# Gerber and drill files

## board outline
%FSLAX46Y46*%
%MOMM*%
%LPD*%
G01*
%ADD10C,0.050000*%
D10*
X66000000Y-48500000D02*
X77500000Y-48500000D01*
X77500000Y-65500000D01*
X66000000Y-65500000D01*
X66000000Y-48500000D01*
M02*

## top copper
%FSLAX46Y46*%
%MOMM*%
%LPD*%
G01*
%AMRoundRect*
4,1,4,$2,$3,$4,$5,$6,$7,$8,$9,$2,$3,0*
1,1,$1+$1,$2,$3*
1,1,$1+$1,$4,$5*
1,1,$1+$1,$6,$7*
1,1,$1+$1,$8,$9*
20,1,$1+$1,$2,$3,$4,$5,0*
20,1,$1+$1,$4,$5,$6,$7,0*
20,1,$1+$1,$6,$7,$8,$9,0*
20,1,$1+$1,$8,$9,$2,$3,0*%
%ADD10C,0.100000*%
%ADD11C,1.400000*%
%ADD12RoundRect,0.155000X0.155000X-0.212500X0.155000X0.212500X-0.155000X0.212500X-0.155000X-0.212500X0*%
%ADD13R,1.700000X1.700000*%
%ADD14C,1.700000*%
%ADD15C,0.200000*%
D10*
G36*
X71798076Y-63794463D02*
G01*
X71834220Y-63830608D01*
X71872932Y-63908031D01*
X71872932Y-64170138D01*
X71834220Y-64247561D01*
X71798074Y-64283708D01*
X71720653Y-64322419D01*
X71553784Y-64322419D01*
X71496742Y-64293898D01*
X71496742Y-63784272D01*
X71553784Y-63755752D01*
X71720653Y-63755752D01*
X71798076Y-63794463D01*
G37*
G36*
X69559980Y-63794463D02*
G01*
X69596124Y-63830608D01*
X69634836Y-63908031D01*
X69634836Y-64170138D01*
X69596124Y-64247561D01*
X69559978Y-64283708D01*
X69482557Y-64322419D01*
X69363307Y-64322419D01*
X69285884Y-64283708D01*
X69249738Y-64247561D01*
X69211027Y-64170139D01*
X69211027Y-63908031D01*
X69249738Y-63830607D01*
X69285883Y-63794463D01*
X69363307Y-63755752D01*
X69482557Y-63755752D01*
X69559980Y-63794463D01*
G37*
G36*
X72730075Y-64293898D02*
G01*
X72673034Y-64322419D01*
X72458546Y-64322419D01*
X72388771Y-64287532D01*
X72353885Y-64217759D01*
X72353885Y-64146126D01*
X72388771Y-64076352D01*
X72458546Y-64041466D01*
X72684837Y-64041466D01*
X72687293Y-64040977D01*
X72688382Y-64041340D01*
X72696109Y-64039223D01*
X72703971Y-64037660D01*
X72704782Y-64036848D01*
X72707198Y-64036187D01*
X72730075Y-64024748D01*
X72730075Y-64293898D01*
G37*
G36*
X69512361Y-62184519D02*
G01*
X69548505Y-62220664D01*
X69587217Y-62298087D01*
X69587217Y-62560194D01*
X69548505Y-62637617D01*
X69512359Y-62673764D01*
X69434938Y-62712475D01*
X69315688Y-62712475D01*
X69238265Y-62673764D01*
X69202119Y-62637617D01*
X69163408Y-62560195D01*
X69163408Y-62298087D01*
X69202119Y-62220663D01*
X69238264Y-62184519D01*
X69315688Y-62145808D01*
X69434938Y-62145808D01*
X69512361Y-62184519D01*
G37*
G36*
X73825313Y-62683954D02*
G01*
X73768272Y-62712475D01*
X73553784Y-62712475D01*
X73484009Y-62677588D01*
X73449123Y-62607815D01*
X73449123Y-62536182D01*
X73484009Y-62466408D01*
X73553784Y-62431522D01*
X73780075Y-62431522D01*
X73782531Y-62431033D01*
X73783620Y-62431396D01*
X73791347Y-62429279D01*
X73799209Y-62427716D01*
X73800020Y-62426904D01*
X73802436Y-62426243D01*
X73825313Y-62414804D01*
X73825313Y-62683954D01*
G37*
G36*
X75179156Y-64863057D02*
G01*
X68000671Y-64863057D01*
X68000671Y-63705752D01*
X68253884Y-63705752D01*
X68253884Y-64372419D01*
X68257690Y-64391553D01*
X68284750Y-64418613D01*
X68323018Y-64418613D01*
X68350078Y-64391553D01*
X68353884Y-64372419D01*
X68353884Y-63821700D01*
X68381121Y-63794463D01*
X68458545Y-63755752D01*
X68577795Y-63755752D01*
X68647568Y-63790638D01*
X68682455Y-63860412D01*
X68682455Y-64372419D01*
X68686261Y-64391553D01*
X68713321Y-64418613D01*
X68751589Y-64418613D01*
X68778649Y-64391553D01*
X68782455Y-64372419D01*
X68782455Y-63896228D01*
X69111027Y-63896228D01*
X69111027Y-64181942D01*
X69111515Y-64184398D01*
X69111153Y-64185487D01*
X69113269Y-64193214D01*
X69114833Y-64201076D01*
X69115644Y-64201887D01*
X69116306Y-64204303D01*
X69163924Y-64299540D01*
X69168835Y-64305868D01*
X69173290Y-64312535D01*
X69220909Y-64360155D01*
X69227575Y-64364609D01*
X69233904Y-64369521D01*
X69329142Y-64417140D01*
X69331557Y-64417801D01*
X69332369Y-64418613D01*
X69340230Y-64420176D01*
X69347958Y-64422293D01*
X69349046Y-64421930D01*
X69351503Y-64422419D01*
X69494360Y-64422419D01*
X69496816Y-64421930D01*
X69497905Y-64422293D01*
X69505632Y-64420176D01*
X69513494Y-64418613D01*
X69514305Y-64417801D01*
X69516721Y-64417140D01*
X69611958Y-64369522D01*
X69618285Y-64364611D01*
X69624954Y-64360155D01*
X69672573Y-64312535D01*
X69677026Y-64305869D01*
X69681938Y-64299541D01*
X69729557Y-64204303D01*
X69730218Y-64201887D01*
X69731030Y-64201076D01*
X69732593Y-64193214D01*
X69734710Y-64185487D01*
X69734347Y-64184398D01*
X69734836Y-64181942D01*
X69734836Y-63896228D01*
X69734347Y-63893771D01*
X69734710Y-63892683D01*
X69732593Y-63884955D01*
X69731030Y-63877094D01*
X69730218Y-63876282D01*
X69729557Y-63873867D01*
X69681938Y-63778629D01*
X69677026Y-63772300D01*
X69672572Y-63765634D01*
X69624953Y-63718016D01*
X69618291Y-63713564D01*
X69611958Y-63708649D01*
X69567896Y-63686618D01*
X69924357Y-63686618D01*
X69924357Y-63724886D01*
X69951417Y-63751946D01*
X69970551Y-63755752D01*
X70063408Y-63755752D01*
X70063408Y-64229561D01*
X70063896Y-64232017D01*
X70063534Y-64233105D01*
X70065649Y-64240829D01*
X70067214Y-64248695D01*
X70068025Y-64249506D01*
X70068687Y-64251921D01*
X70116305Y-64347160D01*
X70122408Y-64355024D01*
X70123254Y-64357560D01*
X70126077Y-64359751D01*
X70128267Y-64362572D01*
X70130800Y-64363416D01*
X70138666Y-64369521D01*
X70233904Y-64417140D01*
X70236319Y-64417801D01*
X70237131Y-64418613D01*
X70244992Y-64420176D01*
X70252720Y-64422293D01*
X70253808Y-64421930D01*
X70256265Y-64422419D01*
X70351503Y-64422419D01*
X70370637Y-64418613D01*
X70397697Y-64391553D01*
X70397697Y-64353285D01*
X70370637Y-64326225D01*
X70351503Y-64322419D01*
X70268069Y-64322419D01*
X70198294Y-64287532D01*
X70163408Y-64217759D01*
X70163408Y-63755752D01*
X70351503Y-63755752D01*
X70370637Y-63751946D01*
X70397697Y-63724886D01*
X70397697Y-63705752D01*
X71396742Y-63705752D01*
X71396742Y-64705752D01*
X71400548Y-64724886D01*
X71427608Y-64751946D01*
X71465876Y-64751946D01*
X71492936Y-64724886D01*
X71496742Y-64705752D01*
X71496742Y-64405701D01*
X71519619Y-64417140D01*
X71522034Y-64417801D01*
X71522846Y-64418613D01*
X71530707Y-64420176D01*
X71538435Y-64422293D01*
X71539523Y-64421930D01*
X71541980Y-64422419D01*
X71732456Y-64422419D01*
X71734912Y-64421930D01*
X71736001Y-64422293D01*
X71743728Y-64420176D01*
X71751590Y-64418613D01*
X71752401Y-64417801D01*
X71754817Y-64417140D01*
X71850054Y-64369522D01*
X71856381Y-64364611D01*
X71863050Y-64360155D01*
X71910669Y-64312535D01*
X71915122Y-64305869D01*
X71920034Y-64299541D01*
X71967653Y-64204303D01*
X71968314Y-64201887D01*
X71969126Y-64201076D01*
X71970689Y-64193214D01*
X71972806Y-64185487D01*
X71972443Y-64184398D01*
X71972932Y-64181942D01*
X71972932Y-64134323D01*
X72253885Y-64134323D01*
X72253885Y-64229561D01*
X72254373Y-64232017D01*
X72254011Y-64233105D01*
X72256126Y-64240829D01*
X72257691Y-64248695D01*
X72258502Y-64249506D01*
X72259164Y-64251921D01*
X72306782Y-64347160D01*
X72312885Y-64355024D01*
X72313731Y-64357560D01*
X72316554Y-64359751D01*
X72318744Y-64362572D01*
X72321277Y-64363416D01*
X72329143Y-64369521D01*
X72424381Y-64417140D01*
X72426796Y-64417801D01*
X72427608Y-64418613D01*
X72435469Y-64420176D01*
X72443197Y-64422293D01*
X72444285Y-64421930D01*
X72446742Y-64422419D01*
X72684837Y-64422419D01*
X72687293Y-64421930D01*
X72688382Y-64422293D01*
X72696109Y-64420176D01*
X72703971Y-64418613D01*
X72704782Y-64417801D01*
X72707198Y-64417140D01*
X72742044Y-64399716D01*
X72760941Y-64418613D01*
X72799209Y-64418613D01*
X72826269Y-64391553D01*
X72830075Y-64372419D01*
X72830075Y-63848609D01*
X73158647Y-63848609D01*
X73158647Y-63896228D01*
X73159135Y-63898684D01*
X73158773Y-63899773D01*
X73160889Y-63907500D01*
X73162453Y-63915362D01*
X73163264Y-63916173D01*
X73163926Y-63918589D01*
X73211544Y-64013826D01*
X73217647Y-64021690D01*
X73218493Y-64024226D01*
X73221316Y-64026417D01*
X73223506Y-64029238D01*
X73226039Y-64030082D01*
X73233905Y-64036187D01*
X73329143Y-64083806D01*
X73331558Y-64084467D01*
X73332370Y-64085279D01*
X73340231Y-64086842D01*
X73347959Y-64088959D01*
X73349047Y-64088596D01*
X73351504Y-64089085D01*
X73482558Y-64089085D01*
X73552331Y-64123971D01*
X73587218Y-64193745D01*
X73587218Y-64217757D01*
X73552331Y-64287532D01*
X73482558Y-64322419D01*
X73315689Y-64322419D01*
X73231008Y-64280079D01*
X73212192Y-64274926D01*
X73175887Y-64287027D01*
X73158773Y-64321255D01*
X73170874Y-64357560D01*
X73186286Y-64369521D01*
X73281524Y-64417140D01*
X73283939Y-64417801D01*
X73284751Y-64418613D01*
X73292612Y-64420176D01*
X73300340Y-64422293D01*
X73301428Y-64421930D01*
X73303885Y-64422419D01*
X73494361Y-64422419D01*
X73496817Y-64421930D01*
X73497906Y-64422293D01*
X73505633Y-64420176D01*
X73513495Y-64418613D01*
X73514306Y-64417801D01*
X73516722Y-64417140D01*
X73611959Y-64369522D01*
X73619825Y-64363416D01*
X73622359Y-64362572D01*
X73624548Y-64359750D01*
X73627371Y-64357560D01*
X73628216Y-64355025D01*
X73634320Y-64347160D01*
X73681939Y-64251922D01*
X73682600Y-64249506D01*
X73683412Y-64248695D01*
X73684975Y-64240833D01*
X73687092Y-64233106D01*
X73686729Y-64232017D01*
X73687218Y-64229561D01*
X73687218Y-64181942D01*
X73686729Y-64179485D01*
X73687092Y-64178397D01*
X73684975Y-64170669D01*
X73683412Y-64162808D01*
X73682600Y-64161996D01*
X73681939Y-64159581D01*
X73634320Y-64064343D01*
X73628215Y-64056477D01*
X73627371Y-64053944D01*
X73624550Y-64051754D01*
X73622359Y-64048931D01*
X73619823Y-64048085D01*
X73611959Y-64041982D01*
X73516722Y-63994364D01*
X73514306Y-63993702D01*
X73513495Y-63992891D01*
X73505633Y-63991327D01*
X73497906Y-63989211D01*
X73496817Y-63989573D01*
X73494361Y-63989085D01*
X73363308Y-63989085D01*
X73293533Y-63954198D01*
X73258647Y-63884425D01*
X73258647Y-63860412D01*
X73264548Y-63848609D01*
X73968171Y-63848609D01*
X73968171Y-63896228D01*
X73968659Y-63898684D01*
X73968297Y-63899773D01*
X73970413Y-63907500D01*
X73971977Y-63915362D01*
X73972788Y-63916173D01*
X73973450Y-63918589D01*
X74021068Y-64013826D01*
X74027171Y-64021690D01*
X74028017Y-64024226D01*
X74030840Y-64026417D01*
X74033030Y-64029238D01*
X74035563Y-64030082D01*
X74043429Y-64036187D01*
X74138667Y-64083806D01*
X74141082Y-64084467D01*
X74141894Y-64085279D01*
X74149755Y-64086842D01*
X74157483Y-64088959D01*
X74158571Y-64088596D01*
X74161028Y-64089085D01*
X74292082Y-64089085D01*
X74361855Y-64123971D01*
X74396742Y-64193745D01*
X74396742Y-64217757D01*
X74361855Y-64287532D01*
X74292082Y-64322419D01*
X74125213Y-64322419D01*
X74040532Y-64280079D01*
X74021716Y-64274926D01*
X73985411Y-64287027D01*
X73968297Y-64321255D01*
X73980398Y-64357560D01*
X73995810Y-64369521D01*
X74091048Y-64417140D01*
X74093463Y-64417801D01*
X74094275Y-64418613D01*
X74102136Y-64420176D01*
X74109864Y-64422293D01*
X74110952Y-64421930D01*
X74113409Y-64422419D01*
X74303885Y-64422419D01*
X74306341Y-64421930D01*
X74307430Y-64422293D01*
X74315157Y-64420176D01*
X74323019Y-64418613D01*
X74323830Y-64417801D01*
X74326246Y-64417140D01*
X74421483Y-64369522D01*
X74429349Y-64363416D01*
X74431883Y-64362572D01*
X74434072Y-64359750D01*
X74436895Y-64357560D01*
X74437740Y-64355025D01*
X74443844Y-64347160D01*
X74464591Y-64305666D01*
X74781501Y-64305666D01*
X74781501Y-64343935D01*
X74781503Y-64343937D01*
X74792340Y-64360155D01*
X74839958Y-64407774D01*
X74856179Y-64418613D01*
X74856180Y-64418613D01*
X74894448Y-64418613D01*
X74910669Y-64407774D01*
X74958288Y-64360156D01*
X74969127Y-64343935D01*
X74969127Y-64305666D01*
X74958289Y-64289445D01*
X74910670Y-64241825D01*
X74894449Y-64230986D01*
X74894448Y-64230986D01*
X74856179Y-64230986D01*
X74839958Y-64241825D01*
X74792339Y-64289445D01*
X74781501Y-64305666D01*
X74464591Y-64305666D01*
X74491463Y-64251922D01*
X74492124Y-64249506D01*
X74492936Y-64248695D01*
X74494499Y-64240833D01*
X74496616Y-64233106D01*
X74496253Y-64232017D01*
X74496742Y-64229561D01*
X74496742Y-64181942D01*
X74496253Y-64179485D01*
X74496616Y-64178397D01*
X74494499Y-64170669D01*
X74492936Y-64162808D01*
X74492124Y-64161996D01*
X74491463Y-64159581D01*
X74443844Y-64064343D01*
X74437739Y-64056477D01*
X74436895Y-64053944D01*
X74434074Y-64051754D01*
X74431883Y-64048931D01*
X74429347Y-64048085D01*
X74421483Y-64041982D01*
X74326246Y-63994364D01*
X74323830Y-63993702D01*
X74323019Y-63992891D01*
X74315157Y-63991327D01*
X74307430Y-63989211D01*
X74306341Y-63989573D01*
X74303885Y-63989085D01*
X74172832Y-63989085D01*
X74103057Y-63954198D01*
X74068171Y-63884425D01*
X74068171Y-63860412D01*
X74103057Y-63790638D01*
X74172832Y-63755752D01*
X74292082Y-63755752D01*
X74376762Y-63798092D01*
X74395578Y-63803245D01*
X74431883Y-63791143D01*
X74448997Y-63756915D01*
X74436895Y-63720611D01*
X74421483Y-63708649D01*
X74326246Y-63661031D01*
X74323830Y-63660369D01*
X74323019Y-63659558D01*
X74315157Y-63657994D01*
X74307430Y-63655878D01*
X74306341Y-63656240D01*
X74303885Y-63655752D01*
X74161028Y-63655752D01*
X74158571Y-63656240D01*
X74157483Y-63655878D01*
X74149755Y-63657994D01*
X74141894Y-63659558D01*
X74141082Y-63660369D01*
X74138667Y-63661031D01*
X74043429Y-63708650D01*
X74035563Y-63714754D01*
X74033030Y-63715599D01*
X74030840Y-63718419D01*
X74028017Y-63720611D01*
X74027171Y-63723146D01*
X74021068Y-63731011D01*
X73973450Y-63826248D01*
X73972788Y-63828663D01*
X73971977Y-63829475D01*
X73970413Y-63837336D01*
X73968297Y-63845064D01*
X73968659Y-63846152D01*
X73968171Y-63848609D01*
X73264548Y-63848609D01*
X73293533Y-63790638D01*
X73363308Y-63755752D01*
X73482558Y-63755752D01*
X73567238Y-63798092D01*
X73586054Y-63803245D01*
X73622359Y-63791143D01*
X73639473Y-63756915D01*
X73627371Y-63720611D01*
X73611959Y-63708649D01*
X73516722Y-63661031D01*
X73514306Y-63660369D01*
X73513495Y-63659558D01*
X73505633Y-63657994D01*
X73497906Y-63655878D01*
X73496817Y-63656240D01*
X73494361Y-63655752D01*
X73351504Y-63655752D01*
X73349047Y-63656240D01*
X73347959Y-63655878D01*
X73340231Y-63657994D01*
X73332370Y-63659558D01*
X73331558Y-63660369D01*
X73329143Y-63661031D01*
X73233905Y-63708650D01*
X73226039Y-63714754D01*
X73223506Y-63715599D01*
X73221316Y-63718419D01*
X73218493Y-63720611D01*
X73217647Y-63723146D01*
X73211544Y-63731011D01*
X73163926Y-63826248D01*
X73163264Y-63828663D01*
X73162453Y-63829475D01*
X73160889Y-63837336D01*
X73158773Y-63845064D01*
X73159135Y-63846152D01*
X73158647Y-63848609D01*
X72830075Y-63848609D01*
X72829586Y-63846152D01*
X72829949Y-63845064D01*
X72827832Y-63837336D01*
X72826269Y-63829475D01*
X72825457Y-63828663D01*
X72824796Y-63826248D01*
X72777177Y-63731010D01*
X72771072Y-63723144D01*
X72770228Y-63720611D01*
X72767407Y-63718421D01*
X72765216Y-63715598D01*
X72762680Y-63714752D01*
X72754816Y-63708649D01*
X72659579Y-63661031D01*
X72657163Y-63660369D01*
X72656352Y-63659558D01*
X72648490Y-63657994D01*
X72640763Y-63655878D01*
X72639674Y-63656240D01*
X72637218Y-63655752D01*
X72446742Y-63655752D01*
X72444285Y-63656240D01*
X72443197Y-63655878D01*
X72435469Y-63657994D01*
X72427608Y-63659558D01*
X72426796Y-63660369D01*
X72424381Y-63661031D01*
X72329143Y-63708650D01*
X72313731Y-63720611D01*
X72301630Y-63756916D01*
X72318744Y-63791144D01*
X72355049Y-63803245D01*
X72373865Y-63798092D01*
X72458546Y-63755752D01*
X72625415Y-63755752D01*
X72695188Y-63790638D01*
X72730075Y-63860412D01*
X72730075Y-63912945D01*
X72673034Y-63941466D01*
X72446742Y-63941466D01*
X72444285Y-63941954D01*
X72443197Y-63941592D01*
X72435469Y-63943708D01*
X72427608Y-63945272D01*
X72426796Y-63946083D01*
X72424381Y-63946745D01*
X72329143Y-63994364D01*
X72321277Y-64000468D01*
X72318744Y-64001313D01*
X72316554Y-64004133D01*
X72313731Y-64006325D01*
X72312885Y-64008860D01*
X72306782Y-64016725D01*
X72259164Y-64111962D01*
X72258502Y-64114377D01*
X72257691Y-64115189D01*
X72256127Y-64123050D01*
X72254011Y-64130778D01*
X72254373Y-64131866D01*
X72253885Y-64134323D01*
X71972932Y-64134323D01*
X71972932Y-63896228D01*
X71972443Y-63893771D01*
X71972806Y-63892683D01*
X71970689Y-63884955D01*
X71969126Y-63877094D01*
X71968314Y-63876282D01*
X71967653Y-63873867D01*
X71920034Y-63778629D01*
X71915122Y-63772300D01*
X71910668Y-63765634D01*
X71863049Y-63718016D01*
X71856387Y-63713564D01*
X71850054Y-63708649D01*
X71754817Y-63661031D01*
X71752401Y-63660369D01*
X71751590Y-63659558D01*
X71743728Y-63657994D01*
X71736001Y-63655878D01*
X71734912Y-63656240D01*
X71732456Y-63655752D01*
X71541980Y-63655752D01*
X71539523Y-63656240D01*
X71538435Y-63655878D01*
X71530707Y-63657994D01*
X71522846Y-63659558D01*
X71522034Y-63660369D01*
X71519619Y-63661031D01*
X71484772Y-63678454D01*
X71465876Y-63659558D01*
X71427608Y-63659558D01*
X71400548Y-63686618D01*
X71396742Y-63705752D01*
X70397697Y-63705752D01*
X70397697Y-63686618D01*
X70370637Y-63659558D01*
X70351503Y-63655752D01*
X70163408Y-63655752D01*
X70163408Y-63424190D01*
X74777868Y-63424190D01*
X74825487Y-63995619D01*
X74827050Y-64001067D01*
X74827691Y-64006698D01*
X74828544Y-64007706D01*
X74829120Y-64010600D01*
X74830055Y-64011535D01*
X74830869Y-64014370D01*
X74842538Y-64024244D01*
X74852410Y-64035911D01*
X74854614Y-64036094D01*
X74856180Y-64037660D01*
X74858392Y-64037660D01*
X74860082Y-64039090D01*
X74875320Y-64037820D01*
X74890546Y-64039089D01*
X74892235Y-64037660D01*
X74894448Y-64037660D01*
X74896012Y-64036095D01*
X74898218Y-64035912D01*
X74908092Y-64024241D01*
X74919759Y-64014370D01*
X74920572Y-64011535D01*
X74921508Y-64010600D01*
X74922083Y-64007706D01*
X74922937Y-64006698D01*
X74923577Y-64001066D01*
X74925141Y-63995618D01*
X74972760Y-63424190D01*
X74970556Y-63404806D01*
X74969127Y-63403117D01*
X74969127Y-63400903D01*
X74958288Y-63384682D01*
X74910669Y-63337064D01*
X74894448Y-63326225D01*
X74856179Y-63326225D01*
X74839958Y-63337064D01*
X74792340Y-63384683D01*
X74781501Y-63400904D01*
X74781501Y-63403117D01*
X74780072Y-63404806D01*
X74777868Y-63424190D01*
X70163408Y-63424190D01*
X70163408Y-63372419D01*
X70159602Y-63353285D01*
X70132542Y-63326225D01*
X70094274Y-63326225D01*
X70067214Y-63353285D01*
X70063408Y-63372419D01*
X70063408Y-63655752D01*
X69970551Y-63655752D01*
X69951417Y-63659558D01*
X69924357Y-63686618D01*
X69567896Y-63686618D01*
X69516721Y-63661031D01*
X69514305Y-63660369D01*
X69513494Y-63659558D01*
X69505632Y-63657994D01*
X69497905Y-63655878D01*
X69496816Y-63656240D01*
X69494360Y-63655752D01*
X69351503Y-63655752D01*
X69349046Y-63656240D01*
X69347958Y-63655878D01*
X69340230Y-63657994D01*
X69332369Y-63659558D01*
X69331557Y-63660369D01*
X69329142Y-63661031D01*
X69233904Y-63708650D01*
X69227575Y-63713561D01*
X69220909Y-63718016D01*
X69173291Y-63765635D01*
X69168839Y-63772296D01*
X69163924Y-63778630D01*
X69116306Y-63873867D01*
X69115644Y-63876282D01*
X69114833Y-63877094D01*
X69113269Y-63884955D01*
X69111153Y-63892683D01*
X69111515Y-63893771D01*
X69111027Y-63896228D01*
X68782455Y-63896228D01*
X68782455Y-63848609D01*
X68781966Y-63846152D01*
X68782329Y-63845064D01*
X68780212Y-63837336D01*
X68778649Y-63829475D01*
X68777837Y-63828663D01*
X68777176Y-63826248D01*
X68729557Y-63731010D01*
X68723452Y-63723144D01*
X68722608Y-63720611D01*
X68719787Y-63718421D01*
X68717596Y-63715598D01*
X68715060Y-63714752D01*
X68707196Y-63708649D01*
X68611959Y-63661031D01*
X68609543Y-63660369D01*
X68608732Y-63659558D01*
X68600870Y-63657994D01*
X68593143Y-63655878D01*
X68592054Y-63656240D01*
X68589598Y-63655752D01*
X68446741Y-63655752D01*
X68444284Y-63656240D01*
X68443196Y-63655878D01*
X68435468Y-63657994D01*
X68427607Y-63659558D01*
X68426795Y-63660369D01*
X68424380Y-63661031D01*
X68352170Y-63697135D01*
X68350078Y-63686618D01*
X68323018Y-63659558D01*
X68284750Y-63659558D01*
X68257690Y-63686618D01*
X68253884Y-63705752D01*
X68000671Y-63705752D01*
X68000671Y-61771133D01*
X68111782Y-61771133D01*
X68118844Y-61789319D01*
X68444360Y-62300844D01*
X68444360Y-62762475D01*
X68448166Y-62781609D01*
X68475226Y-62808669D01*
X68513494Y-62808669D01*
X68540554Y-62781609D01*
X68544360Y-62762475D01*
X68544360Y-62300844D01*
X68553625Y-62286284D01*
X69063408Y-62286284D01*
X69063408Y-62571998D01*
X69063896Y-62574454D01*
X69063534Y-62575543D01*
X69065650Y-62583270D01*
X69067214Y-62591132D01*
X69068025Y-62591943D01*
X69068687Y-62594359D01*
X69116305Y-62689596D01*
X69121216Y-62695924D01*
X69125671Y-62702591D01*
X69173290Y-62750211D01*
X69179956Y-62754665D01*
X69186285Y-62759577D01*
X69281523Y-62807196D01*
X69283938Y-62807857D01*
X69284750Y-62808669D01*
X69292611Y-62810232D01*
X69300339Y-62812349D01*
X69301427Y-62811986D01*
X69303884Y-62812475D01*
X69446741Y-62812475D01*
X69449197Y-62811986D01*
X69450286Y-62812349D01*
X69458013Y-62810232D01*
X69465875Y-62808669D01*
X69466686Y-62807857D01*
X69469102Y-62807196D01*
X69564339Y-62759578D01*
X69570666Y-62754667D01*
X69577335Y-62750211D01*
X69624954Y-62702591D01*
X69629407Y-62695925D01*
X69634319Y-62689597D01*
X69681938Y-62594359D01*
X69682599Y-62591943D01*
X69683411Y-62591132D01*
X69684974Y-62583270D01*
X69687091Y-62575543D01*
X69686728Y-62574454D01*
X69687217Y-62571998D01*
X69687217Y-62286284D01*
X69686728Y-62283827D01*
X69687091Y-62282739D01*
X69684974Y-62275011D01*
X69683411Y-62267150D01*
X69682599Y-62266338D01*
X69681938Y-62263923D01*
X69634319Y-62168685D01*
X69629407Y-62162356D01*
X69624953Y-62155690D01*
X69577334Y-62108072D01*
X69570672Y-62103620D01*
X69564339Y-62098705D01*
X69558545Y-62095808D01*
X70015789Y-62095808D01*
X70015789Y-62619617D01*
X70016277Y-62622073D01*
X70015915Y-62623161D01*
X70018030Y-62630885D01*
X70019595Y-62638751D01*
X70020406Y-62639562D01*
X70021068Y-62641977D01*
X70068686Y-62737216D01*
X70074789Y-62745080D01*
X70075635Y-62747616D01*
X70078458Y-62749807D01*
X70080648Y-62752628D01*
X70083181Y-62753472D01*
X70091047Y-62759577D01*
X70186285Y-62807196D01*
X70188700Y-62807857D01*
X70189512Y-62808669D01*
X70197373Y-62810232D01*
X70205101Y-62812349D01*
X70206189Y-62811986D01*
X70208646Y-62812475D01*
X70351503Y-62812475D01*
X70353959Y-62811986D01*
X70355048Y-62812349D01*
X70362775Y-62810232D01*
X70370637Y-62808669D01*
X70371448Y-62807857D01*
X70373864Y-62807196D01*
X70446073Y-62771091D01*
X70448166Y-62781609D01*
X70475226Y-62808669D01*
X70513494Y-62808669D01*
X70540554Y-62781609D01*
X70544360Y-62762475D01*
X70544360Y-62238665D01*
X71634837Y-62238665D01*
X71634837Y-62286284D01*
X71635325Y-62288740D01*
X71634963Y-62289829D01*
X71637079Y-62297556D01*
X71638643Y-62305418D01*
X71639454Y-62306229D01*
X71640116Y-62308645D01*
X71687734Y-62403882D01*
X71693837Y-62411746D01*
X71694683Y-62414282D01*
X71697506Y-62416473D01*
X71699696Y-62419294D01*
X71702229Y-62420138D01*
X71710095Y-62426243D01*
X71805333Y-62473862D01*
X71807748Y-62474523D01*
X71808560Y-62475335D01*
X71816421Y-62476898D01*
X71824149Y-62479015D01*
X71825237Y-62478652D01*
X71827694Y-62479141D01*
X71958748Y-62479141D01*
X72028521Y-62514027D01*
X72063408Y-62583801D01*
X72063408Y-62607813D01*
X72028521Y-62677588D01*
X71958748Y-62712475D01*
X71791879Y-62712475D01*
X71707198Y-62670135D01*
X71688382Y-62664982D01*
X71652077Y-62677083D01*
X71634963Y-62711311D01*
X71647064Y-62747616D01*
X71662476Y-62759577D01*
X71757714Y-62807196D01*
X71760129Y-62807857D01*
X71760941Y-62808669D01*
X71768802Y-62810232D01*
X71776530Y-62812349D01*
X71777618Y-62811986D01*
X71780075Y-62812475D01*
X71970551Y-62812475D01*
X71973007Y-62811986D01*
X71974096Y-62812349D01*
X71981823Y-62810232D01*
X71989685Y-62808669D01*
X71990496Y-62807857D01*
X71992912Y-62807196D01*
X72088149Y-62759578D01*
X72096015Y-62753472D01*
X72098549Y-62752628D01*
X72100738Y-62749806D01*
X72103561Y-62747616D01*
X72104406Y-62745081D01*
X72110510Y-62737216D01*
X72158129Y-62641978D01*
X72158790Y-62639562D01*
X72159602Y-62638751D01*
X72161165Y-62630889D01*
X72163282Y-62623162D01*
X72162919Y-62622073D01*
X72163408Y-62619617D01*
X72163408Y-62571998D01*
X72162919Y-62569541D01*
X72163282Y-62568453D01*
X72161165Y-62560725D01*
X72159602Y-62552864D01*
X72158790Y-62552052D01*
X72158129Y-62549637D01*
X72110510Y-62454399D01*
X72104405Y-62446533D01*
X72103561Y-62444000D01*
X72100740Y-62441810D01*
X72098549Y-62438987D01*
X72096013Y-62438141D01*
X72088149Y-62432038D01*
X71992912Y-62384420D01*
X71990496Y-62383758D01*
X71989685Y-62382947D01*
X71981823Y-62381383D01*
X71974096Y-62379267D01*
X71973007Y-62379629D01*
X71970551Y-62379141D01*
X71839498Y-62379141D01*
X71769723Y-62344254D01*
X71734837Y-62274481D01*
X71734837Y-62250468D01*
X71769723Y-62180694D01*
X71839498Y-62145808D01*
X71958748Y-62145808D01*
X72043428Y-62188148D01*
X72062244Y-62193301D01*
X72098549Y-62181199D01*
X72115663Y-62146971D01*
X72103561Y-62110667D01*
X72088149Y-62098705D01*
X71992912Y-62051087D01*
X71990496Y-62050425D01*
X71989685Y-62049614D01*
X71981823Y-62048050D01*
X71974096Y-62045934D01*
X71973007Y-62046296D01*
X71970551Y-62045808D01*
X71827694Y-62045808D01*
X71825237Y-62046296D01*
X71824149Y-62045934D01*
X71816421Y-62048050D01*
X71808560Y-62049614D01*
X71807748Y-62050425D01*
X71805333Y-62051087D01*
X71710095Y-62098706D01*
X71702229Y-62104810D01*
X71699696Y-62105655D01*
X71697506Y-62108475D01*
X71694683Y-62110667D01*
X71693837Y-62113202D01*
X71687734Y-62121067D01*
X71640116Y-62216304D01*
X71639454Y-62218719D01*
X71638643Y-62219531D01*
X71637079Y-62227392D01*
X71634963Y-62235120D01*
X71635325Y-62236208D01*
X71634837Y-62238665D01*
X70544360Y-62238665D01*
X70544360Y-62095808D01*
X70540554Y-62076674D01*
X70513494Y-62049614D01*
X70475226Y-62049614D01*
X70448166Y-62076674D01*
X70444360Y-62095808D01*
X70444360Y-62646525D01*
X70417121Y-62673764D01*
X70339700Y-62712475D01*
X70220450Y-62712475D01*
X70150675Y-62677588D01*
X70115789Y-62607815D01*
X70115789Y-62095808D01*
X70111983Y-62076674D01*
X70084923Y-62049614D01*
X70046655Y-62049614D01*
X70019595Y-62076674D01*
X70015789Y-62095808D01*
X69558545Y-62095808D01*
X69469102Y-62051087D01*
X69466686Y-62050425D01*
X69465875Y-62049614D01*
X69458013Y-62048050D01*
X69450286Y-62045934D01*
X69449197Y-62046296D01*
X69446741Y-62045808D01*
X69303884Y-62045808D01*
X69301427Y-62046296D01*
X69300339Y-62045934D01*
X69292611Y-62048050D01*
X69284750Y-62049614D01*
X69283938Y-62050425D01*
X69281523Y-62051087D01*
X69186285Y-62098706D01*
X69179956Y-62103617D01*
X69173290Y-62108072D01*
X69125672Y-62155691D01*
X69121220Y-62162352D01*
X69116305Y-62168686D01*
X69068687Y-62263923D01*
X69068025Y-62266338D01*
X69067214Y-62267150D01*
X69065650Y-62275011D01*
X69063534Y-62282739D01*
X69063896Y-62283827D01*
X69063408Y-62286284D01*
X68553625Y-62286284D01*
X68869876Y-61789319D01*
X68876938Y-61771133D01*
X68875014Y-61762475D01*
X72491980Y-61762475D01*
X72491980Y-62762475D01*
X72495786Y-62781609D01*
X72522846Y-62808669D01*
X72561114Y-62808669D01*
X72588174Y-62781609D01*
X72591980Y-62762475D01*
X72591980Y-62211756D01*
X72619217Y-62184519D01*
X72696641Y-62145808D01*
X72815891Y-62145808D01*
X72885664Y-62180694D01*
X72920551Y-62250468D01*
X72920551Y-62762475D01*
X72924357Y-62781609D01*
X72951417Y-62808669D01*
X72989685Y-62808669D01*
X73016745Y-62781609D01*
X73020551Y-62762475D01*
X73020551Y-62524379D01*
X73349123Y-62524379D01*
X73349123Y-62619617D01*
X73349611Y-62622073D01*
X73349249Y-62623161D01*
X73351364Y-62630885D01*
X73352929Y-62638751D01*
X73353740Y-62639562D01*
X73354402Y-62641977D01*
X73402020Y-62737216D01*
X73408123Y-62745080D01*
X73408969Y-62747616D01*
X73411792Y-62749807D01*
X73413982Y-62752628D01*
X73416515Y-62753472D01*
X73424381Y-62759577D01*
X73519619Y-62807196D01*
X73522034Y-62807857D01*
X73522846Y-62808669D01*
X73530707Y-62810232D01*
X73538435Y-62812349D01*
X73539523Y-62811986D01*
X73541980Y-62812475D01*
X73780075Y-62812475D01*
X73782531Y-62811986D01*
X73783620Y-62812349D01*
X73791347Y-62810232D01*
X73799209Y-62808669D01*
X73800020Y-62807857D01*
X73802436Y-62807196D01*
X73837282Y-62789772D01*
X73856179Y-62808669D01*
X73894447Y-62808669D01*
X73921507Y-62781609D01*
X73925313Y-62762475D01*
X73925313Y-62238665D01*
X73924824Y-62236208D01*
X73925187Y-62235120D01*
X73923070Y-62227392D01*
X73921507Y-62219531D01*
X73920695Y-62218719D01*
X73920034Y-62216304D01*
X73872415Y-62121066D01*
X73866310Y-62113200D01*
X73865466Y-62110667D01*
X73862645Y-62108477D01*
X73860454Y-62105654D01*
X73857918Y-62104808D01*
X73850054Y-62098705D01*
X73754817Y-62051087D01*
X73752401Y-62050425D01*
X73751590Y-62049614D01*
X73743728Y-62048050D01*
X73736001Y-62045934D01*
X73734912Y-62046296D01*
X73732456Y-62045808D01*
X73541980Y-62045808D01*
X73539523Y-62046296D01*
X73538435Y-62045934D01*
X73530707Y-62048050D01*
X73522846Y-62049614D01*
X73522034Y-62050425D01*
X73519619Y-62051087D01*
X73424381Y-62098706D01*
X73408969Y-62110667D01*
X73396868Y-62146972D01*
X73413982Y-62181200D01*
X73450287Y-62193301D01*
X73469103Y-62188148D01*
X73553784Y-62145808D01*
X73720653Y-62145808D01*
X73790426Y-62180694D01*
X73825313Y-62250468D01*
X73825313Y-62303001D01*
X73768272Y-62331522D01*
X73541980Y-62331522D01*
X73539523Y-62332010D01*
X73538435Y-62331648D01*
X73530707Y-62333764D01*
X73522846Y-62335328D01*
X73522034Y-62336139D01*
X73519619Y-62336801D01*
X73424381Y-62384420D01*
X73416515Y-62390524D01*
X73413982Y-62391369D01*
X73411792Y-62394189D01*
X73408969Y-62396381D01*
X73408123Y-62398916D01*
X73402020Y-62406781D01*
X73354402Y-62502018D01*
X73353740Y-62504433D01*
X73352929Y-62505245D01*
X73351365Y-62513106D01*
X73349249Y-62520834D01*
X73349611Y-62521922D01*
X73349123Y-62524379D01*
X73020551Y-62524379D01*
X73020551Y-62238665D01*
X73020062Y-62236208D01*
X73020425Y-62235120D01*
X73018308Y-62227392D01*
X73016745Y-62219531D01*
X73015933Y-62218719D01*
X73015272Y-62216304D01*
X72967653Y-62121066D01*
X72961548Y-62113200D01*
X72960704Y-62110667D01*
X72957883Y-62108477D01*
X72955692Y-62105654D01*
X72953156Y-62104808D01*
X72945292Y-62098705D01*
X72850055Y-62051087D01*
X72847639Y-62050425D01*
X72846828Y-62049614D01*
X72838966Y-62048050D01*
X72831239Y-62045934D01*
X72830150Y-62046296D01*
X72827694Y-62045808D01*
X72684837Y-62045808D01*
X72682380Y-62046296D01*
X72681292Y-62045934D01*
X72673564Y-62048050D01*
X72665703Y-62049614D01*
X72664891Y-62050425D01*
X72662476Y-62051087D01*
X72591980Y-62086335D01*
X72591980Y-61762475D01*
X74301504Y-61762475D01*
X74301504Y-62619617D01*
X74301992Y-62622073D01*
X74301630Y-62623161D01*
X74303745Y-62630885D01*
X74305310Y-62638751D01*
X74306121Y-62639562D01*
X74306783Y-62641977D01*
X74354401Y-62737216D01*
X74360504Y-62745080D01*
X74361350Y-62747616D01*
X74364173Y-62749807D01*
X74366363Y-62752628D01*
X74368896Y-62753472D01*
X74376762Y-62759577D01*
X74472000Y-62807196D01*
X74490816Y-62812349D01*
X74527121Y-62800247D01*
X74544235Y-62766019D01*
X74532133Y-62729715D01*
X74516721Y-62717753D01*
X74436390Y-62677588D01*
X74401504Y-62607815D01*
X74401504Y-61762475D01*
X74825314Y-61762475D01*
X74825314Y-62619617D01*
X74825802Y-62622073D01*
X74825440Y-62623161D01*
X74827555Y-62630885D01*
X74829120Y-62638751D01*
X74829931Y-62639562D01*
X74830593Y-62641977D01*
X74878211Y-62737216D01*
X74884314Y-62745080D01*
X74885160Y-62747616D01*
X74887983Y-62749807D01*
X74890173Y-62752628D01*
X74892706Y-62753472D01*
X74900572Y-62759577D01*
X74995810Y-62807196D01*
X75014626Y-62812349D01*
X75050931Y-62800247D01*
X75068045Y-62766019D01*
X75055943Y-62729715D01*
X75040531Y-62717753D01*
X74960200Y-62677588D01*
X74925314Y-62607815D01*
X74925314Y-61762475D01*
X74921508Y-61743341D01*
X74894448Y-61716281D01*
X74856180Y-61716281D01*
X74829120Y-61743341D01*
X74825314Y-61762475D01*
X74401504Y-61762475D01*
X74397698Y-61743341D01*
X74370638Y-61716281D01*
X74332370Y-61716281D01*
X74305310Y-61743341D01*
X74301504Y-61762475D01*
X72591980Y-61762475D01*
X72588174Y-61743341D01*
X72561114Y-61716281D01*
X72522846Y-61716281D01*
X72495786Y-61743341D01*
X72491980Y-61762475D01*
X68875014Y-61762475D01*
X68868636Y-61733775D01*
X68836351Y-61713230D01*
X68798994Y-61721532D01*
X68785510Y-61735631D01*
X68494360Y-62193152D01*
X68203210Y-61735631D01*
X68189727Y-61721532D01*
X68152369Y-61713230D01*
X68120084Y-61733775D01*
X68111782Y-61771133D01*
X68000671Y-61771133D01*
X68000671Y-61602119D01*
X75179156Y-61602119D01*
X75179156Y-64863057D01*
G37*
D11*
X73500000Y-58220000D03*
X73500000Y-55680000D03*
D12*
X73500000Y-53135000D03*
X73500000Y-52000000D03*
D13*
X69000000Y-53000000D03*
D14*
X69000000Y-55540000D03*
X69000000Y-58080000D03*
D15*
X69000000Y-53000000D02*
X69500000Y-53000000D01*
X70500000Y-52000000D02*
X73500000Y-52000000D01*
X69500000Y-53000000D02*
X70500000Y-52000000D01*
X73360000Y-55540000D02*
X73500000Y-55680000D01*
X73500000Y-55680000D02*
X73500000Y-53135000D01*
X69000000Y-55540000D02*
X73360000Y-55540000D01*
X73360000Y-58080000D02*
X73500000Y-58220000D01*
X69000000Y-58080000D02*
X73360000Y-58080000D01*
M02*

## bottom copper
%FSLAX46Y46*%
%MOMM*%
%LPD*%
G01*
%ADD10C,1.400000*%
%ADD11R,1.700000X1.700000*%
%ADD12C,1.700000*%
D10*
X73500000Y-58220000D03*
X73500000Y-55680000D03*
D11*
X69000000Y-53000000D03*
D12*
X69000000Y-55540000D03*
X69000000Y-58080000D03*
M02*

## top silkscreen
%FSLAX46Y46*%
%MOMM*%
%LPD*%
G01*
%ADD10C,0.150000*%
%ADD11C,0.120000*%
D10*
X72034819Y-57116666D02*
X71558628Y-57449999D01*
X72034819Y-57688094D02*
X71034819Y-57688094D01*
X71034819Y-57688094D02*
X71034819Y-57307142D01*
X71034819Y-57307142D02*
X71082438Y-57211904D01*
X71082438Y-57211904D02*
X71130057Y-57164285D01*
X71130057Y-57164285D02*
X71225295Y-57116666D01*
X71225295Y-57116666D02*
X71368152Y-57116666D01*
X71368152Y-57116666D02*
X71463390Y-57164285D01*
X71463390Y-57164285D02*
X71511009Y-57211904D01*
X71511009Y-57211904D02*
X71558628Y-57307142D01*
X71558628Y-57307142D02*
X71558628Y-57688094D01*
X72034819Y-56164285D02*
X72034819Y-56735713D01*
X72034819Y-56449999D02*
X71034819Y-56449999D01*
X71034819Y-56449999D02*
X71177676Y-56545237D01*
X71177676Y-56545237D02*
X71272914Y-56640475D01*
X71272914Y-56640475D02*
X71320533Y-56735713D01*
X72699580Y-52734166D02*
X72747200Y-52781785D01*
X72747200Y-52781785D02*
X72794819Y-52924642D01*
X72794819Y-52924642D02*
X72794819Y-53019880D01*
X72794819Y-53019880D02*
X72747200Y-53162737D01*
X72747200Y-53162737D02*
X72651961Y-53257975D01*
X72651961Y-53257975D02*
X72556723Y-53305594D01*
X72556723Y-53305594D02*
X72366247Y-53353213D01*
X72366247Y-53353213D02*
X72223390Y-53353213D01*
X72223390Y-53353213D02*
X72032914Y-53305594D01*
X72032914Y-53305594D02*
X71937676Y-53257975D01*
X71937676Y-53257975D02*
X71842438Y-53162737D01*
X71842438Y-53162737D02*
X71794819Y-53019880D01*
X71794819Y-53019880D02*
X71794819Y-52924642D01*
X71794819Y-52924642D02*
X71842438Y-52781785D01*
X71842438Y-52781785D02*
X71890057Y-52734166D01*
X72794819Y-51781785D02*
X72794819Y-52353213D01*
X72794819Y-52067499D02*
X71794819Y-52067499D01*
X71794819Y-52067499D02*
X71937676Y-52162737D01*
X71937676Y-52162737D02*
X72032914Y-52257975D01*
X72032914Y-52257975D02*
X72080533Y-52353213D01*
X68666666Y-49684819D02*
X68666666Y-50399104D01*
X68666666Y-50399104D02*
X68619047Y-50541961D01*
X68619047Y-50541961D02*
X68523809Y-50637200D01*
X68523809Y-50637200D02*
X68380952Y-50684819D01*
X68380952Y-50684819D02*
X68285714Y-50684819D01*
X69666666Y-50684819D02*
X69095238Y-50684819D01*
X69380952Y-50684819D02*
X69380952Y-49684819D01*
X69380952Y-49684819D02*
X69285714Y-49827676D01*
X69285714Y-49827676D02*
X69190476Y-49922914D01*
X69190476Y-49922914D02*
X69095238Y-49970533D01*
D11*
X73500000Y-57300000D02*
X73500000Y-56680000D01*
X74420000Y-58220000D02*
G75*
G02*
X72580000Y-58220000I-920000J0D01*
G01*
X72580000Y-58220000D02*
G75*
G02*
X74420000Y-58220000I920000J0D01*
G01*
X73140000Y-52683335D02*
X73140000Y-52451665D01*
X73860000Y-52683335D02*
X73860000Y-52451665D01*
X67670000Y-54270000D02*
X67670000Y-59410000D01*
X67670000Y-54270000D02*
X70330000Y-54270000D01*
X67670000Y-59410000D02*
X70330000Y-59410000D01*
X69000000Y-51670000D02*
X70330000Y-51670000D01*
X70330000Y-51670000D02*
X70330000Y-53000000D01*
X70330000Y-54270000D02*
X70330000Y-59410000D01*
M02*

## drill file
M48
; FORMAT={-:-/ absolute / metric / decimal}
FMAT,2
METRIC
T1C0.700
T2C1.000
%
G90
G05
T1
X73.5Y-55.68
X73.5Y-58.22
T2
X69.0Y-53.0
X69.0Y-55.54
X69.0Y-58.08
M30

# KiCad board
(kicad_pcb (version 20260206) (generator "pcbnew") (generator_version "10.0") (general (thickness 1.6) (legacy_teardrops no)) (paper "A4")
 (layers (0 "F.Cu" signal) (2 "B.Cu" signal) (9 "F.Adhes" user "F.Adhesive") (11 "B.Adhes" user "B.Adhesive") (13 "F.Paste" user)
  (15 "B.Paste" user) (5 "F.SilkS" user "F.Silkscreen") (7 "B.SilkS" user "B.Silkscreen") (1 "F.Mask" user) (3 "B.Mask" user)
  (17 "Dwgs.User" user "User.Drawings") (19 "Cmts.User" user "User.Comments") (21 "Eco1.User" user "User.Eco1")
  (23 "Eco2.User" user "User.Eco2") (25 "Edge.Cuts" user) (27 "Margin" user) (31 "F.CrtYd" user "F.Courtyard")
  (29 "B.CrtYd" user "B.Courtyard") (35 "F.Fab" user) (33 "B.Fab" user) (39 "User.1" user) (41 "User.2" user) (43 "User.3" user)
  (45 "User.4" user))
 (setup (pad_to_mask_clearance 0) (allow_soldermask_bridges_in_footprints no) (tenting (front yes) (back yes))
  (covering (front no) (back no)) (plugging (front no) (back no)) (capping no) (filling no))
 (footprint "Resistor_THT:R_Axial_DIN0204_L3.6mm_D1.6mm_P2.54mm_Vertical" (layer "F.Cu") (at 73.5 58.22 90)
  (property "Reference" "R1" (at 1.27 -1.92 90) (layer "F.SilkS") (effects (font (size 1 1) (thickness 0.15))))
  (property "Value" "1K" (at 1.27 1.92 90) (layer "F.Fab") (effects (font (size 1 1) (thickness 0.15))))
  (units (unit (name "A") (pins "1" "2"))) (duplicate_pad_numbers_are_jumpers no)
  (fp_line (start 0.92 0) (end 1.54 0) (stroke (width 0.12) (type solid)) (layer "F.SilkS"))
  (fp_circle (center 0 0) (end 0.92 0) (stroke (width 0.12) (type solid)) (fill no) (layer "F.SilkS"))
  (pad "1" thru_hole circle (at 0 0 90) (size 1.4 1.4) (drill 0.7) (layers "*.Cu" "*.Mask") (remove_unused_layers no) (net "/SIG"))
  (pad "2" thru_hole circle (at 2.54 0 90) (size 1.4 1.4) (drill 0.7) (layers "*.Cu" "*.Mask") (remove_unused_layers no) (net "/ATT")))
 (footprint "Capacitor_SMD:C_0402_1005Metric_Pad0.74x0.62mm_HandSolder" (layer "F.Cu") (at 73.5 52.5675 90)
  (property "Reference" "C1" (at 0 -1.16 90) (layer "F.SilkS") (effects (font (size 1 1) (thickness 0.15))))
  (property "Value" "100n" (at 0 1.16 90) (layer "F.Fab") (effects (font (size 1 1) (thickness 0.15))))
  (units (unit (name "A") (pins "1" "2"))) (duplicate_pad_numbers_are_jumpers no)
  (fp_line (start -0.115835 -0.36) (end 0.115835 -0.36) (stroke (width 0.12) (type solid)) (layer "F.SilkS"))
  (fp_line (start -0.115835 0.36) (end 0.115835 0.36) (stroke (width 0.12) (type solid)) (layer "F.SilkS"))
  (pad "1" smd roundrect (at -0.5675 0 90) (size 0.735 0.62) (layers "F.Cu" "F.Mask" "F.Paste") (roundrect_rratio 0.25) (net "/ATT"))
  (pad "2" smd roundrect (at 0.5675 0 90) (size 0.735 0.62) (layers "F.Cu" "F.Mask" "F.Paste") (roundrect_rratio 0.25) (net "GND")))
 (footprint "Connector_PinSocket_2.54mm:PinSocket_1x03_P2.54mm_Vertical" (layer "F.Cu") (at 69 53)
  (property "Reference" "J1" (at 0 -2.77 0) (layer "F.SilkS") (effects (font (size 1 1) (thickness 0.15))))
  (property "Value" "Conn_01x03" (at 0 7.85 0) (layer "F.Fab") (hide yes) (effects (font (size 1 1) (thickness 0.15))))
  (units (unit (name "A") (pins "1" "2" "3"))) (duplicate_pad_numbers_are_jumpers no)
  (fp_line (start -1.33 1.27) (end -1.33 6.41) (stroke (width 0.12) (type solid)) (layer "F.SilkS"))
  (fp_line (start -1.33 1.27) (end 1.33 1.27) (stroke (width 0.12) (type solid)) (layer "F.SilkS"))
  (fp_line (start -1.33 6.41) (end 1.33 6.41) (stroke (width 0.12) (type solid)) (layer "F.SilkS"))
  (fp_line (start 0 -1.33) (end 1.33 -1.33) (stroke (width 0.12) (type solid)) (layer "F.SilkS"))
  (fp_line (start 1.33 -1.33) (end 1.33 0) (stroke (width 0.12) (type solid)) (layer "F.SilkS"))
  (fp_line (start 1.33 1.27) (end 1.33 6.41) (stroke (width 0.12) (type solid)) (layer "F.SilkS"))
  (pad "1" thru_hole rect (at 0 0) (size 1.7 1.7) (drill 1) (layers "*.Cu" "*.Mask") (remove_unused_layers no) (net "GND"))
  (pad "2" thru_hole circle (at 0 2.54) (size 1.7 1.7) (drill 1) (layers "*.Cu" "*.Mask") (remove_unused_layers no) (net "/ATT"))
  (pad "3" thru_hole circle (at 0 5.08) (size 1.7 1.7) (drill 1) (layers "*.Cu" "*.Mask") (remove_unused_layers no) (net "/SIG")))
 (gr_rect (start 66 48.5) (end 77.5 65.5) (stroke (width 0.05) (type default)) (fill no) (layer "Edge.Cuts"))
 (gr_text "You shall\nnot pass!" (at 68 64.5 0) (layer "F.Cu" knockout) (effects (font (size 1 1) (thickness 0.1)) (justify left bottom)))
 (segment (start 69 53) (end 69.5 53) (width 0.2) (layer "F.Cu") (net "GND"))
 (segment (start 70.5 52) (end 73.5 52) (width 0.2) (layer "F.Cu") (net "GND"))
 (segment (start 69.5 53) (end 70.5 52) (width 0.2) (layer "F.Cu") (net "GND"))
 (segment (start 73.36 55.54) (end 73.5 55.68) (width 0.2) (layer "F.Cu") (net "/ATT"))
 (segment (start 73.5 55.68) (end 73.5 53.135) (width 0.2) (layer "F.Cu") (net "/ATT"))
 (segment (start 69 55.54) (end 73.36 55.54) (width 0.2) (layer "F.Cu") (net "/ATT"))
 (segment (start 73.36 58.08) (end 73.5 58.22) (width 0.2) (layer "F.Cu") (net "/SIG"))
 (segment (start 69 58.08) (end 73.36 58.08) (width 0.2) (layer "F.Cu") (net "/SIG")))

